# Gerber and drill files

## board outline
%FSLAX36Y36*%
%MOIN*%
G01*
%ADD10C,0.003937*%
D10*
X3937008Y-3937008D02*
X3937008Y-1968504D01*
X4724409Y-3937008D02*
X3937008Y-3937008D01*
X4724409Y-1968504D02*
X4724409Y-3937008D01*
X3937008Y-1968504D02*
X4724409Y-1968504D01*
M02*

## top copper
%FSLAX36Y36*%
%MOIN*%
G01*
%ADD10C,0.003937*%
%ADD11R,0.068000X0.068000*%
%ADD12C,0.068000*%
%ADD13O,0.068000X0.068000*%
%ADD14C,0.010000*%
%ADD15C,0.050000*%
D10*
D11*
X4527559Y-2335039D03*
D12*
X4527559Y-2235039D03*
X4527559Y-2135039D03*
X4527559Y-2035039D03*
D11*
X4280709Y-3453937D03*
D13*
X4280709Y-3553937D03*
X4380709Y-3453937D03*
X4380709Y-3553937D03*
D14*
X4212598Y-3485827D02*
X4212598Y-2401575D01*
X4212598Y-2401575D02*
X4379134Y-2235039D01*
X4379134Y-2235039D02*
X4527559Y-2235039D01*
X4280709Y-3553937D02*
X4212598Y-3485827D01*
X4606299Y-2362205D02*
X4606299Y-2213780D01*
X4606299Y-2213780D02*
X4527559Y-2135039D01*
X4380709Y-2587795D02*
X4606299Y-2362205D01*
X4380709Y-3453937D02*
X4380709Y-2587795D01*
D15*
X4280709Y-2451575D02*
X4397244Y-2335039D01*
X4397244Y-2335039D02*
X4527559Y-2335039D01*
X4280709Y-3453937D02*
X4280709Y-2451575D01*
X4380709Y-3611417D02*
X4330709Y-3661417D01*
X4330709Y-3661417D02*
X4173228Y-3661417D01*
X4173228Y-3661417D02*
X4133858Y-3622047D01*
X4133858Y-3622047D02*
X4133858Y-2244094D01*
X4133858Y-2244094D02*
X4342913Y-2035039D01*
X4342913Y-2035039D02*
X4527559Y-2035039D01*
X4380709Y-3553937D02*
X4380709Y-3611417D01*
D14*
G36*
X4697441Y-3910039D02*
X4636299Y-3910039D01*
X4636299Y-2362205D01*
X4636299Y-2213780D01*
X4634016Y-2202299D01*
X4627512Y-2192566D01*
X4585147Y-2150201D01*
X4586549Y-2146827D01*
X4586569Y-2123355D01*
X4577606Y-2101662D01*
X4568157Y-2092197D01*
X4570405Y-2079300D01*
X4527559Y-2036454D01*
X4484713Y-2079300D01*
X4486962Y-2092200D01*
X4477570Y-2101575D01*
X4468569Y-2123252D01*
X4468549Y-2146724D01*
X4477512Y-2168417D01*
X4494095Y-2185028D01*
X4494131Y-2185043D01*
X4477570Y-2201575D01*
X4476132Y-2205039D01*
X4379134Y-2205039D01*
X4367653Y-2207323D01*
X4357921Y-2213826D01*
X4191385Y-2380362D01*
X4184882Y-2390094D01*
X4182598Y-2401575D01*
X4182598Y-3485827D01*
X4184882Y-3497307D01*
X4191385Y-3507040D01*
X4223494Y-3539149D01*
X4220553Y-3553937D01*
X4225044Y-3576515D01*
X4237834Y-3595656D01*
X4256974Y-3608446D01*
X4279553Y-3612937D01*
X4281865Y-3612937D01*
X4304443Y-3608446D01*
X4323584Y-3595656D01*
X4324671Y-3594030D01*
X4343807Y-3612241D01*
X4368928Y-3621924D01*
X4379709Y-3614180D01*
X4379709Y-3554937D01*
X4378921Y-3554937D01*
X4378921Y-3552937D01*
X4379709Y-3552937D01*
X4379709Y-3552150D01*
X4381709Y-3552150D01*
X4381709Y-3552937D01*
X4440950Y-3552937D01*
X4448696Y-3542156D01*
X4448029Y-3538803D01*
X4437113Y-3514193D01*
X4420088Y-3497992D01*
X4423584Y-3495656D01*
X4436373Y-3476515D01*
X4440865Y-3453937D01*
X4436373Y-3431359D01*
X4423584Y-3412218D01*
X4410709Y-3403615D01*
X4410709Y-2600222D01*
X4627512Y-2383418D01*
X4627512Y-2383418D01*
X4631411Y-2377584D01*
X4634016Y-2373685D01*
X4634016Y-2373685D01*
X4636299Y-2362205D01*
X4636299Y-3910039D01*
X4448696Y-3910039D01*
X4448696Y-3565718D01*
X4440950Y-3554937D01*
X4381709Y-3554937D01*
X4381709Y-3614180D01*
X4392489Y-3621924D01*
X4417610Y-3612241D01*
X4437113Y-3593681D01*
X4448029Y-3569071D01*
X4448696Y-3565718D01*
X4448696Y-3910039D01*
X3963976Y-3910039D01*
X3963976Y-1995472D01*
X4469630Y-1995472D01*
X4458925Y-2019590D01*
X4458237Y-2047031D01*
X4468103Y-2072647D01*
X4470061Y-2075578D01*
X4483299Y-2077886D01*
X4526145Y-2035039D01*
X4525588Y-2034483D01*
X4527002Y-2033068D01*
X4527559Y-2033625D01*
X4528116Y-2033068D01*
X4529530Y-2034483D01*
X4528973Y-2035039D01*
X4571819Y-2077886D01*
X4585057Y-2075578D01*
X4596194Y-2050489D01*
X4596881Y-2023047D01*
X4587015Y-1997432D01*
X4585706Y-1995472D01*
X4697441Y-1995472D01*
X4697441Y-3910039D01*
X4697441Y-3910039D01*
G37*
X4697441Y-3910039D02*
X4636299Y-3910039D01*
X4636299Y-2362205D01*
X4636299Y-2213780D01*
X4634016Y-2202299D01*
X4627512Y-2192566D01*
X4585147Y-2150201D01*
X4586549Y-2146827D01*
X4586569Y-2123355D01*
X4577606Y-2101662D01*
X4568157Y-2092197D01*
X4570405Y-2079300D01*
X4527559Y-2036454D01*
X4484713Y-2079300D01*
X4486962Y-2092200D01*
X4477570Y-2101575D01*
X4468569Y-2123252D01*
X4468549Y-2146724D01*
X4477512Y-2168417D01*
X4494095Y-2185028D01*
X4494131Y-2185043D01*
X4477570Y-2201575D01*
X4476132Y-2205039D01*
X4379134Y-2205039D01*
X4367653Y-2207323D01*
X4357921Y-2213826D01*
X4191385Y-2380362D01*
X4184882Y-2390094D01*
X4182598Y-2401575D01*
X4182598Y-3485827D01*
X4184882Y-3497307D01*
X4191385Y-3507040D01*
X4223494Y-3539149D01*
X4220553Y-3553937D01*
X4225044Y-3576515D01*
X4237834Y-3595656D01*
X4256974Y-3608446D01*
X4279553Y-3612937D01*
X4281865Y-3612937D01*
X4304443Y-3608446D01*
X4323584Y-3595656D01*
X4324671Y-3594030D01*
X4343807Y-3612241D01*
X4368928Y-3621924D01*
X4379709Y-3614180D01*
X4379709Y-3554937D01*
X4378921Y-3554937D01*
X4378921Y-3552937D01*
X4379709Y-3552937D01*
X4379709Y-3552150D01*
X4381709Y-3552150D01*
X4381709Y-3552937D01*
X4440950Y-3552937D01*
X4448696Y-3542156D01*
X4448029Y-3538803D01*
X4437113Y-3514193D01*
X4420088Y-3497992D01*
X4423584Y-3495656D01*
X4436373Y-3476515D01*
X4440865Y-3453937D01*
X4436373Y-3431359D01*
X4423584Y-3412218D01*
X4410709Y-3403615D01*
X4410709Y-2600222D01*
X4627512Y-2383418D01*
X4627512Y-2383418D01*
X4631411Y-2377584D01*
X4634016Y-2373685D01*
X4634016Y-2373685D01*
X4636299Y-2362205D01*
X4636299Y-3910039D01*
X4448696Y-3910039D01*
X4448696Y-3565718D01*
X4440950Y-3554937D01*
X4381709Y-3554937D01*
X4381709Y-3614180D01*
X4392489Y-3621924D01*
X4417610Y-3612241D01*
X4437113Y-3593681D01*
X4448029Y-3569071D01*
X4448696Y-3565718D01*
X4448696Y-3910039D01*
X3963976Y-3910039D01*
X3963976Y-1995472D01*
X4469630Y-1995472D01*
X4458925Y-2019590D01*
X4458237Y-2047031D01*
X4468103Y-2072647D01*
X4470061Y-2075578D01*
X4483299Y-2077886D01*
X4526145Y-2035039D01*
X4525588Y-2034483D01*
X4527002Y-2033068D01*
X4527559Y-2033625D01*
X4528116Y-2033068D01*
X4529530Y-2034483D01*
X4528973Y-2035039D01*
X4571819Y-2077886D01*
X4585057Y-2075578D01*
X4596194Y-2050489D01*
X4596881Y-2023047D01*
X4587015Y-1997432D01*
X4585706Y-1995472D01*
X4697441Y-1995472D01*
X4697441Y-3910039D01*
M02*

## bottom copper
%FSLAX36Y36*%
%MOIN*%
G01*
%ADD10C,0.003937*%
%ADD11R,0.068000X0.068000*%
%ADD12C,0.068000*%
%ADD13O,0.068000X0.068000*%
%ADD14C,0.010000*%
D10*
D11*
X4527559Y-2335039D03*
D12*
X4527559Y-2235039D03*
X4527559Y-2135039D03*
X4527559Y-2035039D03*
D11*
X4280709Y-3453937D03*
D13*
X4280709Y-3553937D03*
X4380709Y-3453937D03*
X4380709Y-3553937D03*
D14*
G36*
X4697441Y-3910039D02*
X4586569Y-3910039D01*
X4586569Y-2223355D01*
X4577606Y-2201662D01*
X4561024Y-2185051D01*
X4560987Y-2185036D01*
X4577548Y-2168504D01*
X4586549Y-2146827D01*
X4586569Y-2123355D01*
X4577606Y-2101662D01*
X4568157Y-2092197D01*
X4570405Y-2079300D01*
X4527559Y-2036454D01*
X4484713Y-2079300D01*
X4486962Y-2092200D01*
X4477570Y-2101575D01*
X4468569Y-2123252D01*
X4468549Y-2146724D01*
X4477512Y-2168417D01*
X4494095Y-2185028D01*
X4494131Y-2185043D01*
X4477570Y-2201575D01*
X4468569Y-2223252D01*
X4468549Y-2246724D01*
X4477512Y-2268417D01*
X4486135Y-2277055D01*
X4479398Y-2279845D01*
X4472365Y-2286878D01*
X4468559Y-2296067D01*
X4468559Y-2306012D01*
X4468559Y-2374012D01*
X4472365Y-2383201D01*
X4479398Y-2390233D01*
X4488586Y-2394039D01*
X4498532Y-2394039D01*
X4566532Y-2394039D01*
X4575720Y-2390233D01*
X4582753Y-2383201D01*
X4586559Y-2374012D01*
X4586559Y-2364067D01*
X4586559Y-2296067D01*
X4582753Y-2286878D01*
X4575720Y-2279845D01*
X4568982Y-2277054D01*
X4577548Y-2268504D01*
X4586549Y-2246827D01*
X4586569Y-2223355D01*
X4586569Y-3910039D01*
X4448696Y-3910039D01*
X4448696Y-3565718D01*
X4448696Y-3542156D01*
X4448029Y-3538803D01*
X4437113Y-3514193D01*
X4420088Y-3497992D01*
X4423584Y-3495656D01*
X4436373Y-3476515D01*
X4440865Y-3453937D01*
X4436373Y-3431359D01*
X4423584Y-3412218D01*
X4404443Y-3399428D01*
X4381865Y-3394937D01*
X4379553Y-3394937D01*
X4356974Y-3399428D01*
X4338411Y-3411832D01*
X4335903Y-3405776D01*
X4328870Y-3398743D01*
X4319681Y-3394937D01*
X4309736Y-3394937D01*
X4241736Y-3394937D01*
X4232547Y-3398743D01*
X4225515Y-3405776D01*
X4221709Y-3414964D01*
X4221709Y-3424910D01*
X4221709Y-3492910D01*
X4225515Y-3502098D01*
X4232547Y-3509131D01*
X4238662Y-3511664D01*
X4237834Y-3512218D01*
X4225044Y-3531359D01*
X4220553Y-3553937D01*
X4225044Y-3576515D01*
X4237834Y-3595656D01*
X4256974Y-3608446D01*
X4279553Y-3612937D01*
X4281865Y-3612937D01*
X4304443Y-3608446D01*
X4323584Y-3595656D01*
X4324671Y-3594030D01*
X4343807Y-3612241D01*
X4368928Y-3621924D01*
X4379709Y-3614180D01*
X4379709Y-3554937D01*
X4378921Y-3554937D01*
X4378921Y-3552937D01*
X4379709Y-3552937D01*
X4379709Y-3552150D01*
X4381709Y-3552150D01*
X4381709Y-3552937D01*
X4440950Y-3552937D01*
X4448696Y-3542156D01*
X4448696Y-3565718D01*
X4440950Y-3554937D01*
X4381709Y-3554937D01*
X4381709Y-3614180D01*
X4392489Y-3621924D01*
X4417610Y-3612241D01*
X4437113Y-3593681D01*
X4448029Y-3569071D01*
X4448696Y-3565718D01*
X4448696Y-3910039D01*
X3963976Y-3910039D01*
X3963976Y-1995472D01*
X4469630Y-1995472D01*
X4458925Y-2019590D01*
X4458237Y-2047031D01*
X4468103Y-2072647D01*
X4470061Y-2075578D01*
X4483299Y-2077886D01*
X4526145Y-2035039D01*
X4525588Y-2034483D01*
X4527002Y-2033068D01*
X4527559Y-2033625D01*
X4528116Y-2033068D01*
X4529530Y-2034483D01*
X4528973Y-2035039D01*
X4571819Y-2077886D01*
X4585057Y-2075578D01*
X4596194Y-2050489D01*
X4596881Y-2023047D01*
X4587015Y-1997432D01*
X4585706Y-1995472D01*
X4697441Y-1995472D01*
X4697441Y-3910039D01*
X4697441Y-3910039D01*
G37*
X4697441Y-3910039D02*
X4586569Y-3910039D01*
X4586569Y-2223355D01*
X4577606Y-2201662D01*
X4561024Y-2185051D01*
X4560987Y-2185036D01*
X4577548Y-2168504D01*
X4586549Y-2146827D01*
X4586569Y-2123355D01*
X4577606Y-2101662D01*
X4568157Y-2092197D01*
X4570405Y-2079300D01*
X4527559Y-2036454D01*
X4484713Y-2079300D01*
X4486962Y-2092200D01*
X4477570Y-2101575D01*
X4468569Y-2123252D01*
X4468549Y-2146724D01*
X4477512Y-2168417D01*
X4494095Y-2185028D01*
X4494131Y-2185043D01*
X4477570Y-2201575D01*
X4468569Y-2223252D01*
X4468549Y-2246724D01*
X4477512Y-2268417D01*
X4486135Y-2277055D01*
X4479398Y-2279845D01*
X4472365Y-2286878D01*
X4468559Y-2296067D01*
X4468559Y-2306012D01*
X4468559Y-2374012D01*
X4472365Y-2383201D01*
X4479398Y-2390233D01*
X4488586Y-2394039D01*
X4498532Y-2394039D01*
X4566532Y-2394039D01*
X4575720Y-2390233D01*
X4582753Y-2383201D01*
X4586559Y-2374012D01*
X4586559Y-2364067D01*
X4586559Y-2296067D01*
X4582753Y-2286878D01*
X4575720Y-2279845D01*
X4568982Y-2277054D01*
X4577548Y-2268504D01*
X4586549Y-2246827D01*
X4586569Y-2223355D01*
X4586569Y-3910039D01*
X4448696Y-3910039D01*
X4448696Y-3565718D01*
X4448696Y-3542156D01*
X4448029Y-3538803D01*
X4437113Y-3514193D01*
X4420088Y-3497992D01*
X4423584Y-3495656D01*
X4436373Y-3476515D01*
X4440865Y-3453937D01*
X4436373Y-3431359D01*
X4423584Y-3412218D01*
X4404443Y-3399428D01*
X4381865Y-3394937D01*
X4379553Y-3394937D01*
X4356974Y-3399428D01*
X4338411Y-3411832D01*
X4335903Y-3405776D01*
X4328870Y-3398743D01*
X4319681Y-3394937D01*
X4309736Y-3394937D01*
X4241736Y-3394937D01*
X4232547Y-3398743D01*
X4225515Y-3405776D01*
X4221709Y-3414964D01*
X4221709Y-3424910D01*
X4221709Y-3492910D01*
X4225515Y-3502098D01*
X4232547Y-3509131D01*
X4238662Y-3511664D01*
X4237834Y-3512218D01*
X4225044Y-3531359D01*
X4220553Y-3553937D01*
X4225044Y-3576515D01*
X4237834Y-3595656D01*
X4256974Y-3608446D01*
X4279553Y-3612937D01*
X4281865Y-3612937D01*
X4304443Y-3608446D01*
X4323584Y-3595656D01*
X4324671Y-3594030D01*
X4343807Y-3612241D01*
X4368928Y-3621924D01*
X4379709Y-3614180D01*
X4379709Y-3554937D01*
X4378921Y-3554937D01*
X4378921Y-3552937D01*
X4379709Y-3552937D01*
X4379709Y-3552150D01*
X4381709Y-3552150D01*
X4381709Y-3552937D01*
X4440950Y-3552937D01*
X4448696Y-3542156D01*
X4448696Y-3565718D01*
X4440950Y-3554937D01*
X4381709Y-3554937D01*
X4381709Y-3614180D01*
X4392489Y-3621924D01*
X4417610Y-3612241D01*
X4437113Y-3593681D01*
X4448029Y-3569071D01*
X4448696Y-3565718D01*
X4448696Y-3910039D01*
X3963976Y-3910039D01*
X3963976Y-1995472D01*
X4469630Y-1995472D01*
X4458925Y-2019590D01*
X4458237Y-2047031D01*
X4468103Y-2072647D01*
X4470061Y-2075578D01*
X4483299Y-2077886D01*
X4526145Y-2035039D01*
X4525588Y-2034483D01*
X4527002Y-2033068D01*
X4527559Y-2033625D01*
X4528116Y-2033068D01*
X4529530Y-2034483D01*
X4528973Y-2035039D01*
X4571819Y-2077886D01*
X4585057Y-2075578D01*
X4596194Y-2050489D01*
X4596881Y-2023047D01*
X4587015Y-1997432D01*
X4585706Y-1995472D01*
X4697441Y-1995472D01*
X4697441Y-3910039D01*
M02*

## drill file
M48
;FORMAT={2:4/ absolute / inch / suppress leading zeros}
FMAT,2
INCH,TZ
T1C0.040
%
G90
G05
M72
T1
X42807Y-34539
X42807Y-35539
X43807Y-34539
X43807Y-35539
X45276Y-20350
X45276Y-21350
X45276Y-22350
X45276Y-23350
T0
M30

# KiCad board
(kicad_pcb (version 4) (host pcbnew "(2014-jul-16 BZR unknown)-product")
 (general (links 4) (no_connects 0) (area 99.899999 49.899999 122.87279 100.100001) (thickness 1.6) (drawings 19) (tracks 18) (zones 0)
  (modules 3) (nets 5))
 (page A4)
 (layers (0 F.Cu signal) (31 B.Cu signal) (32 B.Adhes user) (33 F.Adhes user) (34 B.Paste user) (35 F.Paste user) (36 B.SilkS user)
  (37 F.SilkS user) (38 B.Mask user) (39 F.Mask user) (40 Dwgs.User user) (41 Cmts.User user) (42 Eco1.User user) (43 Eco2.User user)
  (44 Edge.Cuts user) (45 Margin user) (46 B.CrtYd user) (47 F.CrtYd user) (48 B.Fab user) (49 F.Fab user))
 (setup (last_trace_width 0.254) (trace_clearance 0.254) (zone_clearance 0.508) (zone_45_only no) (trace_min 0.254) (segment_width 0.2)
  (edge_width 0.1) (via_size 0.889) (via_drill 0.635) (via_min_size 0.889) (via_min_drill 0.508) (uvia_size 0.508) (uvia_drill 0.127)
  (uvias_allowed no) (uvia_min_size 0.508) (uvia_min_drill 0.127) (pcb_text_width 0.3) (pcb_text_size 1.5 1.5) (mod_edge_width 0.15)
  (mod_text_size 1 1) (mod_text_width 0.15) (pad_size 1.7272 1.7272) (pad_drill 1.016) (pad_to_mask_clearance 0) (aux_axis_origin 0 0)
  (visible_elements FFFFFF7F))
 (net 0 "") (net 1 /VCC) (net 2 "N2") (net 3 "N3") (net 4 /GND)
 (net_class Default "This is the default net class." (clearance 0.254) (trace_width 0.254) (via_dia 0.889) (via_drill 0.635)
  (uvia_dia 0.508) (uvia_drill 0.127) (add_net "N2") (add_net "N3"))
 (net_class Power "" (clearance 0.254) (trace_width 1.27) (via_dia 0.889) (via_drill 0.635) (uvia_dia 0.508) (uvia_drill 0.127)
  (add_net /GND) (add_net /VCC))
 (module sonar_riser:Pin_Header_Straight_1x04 (layer F.Cu) (at 115 55.5 90)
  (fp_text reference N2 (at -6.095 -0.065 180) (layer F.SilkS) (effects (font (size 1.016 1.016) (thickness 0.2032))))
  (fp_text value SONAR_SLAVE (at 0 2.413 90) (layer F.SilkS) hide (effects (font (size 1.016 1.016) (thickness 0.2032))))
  (pad 1 thru_hole rect (at -3.81 0 90) (size 1.7272 1.7272) (drill 1.016) (layers *.Cu *.Mask F.SilkS) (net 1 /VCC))
  (pad 2 thru_hole circle (at -1.27 0 90) (size 1.7272 1.7272) (drill 1.016) (layers *.Cu *.Mask F.SilkS) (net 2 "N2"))
  (pad 3 thru_hole circle (at 1.27 0 90) (size 1.7272 1.7272) (drill 1.016) (layers *.Cu *.Mask F.SilkS) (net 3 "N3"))
  (pad 4 thru_hole circle (at 3.81 0 90) (size 1.7272 1.7272) (drill 1.016) (layers *.Cu *.Mask F.SilkS) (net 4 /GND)))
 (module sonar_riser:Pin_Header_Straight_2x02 (layer B.Cu) (at 110 89)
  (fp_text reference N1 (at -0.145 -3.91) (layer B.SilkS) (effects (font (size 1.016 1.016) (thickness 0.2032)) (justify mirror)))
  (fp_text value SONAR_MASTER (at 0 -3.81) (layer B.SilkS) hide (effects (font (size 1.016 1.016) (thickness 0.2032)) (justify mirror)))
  (pad 1 thru_hole rect (at -1.27 -1.27) (size 1.7272 1.7272) (drill 1.016) (layers *.Cu *.Mask B.SilkS) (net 1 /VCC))
  (pad 2 thru_hole oval (at -1.27 1.27) (size 1.7272 1.7272) (drill 1.016) (layers *.Cu *.Mask B.SilkS) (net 2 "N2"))
  (pad 3 thru_hole oval (at 1.27 -1.27) (size 1.7272 1.7272) (drill 1.016) (layers *.Cu *.Mask B.SilkS) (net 3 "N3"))
  (pad 4 thru_hole oval (at 1.27 1.27) (size 1.7272 1.7272) (drill 1.016) (layers *.Cu *.Mask B.SilkS) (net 4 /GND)))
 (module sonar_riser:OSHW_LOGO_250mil (layer F.Cu) (at 109.855 73.66)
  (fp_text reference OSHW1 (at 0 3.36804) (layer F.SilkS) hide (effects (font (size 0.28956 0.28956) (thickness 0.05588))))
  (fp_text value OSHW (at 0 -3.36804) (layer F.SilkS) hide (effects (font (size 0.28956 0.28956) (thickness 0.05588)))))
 (gr_line (start 100 100) (end 100 50) (angle 90) (layer Edge.Cuts) (width 0.1))
 (gr_line (start 120 100) (end 100 100) (angle 90) (layer Edge.Cuts) (width 0.1))
 (gr_line (start 120 50) (end 120 100) (angle 90) (layer Edge.Cuts) (width 0.1))
 (gr_line (start 100 50) (end 120 50) (angle 90) (layer Edge.Cuts) (width 0.1))
 (segment (start 107 88.54) (end 107 61) (width 0.254) (layer F.Cu) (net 2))
 (segment (start 107 61) (end 111.23 56.77) (width 0.254) (layer F.Cu) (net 2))
 (segment (start 111.23 56.77) (end 115 56.77) (width 0.254) (layer F.Cu) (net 2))
 (segment (start 108.73 90.27) (end 107 88.54) (width 0.254) (layer F.Cu) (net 2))
 (segment (start 117 60) (end 117 56.23) (width 0.254) (layer F.Cu) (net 3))
 (segment (start 117 56.23) (end 115 54.23) (width 0.254) (layer F.Cu) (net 3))
 (segment (start 111.27 65.73) (end 117 60) (width 0.254) (layer F.Cu) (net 3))
 (segment (start 111.27 87.73) (end 111.27 65.73) (width 0.254) (layer F.Cu) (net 3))
 (segment (start 108.73 62.27) (end 111.69 59.31) (width 1.27) (layer F.Cu) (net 1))
 (segment (start 111.69 59.31) (end 115 59.31) (width 1.27) (layer F.Cu) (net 1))
 (segment (start 108.73 87.73) (end 108.73 62.27) (width 1.27) (layer F.Cu) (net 1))
 (segment (start 111.27 91.73) (end 110 93) (width 1.27) (layer F.Cu) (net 4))
 (segment (start 110 93) (end 106 93) (width 1.27) (layer F.Cu) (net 4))
 (segment (start 106 93) (end 105 92) (width 1.27) (layer F.Cu) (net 4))
 (segment (start 105 92) (end 105 57) (width 1.27) (layer F.Cu) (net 4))
 (segment (start 105 57) (end 110.31 51.69) (width 1.27) (layer F.Cu) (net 4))
 (segment (start 110.31 51.69) (end 115 51.69) (width 1.27) (layer F.Cu) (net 4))
 (segment (start 111.27 90.27) (end 111.27 91.73) (width 1.27) (layer F.Cu) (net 4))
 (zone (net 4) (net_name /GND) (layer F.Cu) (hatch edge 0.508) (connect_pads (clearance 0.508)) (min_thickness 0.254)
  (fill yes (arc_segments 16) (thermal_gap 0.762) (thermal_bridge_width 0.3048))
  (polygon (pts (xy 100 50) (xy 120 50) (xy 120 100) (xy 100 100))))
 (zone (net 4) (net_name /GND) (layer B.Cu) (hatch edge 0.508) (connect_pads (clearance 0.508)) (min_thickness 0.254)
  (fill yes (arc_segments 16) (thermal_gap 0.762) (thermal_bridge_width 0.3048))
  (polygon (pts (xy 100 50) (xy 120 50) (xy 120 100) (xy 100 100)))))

